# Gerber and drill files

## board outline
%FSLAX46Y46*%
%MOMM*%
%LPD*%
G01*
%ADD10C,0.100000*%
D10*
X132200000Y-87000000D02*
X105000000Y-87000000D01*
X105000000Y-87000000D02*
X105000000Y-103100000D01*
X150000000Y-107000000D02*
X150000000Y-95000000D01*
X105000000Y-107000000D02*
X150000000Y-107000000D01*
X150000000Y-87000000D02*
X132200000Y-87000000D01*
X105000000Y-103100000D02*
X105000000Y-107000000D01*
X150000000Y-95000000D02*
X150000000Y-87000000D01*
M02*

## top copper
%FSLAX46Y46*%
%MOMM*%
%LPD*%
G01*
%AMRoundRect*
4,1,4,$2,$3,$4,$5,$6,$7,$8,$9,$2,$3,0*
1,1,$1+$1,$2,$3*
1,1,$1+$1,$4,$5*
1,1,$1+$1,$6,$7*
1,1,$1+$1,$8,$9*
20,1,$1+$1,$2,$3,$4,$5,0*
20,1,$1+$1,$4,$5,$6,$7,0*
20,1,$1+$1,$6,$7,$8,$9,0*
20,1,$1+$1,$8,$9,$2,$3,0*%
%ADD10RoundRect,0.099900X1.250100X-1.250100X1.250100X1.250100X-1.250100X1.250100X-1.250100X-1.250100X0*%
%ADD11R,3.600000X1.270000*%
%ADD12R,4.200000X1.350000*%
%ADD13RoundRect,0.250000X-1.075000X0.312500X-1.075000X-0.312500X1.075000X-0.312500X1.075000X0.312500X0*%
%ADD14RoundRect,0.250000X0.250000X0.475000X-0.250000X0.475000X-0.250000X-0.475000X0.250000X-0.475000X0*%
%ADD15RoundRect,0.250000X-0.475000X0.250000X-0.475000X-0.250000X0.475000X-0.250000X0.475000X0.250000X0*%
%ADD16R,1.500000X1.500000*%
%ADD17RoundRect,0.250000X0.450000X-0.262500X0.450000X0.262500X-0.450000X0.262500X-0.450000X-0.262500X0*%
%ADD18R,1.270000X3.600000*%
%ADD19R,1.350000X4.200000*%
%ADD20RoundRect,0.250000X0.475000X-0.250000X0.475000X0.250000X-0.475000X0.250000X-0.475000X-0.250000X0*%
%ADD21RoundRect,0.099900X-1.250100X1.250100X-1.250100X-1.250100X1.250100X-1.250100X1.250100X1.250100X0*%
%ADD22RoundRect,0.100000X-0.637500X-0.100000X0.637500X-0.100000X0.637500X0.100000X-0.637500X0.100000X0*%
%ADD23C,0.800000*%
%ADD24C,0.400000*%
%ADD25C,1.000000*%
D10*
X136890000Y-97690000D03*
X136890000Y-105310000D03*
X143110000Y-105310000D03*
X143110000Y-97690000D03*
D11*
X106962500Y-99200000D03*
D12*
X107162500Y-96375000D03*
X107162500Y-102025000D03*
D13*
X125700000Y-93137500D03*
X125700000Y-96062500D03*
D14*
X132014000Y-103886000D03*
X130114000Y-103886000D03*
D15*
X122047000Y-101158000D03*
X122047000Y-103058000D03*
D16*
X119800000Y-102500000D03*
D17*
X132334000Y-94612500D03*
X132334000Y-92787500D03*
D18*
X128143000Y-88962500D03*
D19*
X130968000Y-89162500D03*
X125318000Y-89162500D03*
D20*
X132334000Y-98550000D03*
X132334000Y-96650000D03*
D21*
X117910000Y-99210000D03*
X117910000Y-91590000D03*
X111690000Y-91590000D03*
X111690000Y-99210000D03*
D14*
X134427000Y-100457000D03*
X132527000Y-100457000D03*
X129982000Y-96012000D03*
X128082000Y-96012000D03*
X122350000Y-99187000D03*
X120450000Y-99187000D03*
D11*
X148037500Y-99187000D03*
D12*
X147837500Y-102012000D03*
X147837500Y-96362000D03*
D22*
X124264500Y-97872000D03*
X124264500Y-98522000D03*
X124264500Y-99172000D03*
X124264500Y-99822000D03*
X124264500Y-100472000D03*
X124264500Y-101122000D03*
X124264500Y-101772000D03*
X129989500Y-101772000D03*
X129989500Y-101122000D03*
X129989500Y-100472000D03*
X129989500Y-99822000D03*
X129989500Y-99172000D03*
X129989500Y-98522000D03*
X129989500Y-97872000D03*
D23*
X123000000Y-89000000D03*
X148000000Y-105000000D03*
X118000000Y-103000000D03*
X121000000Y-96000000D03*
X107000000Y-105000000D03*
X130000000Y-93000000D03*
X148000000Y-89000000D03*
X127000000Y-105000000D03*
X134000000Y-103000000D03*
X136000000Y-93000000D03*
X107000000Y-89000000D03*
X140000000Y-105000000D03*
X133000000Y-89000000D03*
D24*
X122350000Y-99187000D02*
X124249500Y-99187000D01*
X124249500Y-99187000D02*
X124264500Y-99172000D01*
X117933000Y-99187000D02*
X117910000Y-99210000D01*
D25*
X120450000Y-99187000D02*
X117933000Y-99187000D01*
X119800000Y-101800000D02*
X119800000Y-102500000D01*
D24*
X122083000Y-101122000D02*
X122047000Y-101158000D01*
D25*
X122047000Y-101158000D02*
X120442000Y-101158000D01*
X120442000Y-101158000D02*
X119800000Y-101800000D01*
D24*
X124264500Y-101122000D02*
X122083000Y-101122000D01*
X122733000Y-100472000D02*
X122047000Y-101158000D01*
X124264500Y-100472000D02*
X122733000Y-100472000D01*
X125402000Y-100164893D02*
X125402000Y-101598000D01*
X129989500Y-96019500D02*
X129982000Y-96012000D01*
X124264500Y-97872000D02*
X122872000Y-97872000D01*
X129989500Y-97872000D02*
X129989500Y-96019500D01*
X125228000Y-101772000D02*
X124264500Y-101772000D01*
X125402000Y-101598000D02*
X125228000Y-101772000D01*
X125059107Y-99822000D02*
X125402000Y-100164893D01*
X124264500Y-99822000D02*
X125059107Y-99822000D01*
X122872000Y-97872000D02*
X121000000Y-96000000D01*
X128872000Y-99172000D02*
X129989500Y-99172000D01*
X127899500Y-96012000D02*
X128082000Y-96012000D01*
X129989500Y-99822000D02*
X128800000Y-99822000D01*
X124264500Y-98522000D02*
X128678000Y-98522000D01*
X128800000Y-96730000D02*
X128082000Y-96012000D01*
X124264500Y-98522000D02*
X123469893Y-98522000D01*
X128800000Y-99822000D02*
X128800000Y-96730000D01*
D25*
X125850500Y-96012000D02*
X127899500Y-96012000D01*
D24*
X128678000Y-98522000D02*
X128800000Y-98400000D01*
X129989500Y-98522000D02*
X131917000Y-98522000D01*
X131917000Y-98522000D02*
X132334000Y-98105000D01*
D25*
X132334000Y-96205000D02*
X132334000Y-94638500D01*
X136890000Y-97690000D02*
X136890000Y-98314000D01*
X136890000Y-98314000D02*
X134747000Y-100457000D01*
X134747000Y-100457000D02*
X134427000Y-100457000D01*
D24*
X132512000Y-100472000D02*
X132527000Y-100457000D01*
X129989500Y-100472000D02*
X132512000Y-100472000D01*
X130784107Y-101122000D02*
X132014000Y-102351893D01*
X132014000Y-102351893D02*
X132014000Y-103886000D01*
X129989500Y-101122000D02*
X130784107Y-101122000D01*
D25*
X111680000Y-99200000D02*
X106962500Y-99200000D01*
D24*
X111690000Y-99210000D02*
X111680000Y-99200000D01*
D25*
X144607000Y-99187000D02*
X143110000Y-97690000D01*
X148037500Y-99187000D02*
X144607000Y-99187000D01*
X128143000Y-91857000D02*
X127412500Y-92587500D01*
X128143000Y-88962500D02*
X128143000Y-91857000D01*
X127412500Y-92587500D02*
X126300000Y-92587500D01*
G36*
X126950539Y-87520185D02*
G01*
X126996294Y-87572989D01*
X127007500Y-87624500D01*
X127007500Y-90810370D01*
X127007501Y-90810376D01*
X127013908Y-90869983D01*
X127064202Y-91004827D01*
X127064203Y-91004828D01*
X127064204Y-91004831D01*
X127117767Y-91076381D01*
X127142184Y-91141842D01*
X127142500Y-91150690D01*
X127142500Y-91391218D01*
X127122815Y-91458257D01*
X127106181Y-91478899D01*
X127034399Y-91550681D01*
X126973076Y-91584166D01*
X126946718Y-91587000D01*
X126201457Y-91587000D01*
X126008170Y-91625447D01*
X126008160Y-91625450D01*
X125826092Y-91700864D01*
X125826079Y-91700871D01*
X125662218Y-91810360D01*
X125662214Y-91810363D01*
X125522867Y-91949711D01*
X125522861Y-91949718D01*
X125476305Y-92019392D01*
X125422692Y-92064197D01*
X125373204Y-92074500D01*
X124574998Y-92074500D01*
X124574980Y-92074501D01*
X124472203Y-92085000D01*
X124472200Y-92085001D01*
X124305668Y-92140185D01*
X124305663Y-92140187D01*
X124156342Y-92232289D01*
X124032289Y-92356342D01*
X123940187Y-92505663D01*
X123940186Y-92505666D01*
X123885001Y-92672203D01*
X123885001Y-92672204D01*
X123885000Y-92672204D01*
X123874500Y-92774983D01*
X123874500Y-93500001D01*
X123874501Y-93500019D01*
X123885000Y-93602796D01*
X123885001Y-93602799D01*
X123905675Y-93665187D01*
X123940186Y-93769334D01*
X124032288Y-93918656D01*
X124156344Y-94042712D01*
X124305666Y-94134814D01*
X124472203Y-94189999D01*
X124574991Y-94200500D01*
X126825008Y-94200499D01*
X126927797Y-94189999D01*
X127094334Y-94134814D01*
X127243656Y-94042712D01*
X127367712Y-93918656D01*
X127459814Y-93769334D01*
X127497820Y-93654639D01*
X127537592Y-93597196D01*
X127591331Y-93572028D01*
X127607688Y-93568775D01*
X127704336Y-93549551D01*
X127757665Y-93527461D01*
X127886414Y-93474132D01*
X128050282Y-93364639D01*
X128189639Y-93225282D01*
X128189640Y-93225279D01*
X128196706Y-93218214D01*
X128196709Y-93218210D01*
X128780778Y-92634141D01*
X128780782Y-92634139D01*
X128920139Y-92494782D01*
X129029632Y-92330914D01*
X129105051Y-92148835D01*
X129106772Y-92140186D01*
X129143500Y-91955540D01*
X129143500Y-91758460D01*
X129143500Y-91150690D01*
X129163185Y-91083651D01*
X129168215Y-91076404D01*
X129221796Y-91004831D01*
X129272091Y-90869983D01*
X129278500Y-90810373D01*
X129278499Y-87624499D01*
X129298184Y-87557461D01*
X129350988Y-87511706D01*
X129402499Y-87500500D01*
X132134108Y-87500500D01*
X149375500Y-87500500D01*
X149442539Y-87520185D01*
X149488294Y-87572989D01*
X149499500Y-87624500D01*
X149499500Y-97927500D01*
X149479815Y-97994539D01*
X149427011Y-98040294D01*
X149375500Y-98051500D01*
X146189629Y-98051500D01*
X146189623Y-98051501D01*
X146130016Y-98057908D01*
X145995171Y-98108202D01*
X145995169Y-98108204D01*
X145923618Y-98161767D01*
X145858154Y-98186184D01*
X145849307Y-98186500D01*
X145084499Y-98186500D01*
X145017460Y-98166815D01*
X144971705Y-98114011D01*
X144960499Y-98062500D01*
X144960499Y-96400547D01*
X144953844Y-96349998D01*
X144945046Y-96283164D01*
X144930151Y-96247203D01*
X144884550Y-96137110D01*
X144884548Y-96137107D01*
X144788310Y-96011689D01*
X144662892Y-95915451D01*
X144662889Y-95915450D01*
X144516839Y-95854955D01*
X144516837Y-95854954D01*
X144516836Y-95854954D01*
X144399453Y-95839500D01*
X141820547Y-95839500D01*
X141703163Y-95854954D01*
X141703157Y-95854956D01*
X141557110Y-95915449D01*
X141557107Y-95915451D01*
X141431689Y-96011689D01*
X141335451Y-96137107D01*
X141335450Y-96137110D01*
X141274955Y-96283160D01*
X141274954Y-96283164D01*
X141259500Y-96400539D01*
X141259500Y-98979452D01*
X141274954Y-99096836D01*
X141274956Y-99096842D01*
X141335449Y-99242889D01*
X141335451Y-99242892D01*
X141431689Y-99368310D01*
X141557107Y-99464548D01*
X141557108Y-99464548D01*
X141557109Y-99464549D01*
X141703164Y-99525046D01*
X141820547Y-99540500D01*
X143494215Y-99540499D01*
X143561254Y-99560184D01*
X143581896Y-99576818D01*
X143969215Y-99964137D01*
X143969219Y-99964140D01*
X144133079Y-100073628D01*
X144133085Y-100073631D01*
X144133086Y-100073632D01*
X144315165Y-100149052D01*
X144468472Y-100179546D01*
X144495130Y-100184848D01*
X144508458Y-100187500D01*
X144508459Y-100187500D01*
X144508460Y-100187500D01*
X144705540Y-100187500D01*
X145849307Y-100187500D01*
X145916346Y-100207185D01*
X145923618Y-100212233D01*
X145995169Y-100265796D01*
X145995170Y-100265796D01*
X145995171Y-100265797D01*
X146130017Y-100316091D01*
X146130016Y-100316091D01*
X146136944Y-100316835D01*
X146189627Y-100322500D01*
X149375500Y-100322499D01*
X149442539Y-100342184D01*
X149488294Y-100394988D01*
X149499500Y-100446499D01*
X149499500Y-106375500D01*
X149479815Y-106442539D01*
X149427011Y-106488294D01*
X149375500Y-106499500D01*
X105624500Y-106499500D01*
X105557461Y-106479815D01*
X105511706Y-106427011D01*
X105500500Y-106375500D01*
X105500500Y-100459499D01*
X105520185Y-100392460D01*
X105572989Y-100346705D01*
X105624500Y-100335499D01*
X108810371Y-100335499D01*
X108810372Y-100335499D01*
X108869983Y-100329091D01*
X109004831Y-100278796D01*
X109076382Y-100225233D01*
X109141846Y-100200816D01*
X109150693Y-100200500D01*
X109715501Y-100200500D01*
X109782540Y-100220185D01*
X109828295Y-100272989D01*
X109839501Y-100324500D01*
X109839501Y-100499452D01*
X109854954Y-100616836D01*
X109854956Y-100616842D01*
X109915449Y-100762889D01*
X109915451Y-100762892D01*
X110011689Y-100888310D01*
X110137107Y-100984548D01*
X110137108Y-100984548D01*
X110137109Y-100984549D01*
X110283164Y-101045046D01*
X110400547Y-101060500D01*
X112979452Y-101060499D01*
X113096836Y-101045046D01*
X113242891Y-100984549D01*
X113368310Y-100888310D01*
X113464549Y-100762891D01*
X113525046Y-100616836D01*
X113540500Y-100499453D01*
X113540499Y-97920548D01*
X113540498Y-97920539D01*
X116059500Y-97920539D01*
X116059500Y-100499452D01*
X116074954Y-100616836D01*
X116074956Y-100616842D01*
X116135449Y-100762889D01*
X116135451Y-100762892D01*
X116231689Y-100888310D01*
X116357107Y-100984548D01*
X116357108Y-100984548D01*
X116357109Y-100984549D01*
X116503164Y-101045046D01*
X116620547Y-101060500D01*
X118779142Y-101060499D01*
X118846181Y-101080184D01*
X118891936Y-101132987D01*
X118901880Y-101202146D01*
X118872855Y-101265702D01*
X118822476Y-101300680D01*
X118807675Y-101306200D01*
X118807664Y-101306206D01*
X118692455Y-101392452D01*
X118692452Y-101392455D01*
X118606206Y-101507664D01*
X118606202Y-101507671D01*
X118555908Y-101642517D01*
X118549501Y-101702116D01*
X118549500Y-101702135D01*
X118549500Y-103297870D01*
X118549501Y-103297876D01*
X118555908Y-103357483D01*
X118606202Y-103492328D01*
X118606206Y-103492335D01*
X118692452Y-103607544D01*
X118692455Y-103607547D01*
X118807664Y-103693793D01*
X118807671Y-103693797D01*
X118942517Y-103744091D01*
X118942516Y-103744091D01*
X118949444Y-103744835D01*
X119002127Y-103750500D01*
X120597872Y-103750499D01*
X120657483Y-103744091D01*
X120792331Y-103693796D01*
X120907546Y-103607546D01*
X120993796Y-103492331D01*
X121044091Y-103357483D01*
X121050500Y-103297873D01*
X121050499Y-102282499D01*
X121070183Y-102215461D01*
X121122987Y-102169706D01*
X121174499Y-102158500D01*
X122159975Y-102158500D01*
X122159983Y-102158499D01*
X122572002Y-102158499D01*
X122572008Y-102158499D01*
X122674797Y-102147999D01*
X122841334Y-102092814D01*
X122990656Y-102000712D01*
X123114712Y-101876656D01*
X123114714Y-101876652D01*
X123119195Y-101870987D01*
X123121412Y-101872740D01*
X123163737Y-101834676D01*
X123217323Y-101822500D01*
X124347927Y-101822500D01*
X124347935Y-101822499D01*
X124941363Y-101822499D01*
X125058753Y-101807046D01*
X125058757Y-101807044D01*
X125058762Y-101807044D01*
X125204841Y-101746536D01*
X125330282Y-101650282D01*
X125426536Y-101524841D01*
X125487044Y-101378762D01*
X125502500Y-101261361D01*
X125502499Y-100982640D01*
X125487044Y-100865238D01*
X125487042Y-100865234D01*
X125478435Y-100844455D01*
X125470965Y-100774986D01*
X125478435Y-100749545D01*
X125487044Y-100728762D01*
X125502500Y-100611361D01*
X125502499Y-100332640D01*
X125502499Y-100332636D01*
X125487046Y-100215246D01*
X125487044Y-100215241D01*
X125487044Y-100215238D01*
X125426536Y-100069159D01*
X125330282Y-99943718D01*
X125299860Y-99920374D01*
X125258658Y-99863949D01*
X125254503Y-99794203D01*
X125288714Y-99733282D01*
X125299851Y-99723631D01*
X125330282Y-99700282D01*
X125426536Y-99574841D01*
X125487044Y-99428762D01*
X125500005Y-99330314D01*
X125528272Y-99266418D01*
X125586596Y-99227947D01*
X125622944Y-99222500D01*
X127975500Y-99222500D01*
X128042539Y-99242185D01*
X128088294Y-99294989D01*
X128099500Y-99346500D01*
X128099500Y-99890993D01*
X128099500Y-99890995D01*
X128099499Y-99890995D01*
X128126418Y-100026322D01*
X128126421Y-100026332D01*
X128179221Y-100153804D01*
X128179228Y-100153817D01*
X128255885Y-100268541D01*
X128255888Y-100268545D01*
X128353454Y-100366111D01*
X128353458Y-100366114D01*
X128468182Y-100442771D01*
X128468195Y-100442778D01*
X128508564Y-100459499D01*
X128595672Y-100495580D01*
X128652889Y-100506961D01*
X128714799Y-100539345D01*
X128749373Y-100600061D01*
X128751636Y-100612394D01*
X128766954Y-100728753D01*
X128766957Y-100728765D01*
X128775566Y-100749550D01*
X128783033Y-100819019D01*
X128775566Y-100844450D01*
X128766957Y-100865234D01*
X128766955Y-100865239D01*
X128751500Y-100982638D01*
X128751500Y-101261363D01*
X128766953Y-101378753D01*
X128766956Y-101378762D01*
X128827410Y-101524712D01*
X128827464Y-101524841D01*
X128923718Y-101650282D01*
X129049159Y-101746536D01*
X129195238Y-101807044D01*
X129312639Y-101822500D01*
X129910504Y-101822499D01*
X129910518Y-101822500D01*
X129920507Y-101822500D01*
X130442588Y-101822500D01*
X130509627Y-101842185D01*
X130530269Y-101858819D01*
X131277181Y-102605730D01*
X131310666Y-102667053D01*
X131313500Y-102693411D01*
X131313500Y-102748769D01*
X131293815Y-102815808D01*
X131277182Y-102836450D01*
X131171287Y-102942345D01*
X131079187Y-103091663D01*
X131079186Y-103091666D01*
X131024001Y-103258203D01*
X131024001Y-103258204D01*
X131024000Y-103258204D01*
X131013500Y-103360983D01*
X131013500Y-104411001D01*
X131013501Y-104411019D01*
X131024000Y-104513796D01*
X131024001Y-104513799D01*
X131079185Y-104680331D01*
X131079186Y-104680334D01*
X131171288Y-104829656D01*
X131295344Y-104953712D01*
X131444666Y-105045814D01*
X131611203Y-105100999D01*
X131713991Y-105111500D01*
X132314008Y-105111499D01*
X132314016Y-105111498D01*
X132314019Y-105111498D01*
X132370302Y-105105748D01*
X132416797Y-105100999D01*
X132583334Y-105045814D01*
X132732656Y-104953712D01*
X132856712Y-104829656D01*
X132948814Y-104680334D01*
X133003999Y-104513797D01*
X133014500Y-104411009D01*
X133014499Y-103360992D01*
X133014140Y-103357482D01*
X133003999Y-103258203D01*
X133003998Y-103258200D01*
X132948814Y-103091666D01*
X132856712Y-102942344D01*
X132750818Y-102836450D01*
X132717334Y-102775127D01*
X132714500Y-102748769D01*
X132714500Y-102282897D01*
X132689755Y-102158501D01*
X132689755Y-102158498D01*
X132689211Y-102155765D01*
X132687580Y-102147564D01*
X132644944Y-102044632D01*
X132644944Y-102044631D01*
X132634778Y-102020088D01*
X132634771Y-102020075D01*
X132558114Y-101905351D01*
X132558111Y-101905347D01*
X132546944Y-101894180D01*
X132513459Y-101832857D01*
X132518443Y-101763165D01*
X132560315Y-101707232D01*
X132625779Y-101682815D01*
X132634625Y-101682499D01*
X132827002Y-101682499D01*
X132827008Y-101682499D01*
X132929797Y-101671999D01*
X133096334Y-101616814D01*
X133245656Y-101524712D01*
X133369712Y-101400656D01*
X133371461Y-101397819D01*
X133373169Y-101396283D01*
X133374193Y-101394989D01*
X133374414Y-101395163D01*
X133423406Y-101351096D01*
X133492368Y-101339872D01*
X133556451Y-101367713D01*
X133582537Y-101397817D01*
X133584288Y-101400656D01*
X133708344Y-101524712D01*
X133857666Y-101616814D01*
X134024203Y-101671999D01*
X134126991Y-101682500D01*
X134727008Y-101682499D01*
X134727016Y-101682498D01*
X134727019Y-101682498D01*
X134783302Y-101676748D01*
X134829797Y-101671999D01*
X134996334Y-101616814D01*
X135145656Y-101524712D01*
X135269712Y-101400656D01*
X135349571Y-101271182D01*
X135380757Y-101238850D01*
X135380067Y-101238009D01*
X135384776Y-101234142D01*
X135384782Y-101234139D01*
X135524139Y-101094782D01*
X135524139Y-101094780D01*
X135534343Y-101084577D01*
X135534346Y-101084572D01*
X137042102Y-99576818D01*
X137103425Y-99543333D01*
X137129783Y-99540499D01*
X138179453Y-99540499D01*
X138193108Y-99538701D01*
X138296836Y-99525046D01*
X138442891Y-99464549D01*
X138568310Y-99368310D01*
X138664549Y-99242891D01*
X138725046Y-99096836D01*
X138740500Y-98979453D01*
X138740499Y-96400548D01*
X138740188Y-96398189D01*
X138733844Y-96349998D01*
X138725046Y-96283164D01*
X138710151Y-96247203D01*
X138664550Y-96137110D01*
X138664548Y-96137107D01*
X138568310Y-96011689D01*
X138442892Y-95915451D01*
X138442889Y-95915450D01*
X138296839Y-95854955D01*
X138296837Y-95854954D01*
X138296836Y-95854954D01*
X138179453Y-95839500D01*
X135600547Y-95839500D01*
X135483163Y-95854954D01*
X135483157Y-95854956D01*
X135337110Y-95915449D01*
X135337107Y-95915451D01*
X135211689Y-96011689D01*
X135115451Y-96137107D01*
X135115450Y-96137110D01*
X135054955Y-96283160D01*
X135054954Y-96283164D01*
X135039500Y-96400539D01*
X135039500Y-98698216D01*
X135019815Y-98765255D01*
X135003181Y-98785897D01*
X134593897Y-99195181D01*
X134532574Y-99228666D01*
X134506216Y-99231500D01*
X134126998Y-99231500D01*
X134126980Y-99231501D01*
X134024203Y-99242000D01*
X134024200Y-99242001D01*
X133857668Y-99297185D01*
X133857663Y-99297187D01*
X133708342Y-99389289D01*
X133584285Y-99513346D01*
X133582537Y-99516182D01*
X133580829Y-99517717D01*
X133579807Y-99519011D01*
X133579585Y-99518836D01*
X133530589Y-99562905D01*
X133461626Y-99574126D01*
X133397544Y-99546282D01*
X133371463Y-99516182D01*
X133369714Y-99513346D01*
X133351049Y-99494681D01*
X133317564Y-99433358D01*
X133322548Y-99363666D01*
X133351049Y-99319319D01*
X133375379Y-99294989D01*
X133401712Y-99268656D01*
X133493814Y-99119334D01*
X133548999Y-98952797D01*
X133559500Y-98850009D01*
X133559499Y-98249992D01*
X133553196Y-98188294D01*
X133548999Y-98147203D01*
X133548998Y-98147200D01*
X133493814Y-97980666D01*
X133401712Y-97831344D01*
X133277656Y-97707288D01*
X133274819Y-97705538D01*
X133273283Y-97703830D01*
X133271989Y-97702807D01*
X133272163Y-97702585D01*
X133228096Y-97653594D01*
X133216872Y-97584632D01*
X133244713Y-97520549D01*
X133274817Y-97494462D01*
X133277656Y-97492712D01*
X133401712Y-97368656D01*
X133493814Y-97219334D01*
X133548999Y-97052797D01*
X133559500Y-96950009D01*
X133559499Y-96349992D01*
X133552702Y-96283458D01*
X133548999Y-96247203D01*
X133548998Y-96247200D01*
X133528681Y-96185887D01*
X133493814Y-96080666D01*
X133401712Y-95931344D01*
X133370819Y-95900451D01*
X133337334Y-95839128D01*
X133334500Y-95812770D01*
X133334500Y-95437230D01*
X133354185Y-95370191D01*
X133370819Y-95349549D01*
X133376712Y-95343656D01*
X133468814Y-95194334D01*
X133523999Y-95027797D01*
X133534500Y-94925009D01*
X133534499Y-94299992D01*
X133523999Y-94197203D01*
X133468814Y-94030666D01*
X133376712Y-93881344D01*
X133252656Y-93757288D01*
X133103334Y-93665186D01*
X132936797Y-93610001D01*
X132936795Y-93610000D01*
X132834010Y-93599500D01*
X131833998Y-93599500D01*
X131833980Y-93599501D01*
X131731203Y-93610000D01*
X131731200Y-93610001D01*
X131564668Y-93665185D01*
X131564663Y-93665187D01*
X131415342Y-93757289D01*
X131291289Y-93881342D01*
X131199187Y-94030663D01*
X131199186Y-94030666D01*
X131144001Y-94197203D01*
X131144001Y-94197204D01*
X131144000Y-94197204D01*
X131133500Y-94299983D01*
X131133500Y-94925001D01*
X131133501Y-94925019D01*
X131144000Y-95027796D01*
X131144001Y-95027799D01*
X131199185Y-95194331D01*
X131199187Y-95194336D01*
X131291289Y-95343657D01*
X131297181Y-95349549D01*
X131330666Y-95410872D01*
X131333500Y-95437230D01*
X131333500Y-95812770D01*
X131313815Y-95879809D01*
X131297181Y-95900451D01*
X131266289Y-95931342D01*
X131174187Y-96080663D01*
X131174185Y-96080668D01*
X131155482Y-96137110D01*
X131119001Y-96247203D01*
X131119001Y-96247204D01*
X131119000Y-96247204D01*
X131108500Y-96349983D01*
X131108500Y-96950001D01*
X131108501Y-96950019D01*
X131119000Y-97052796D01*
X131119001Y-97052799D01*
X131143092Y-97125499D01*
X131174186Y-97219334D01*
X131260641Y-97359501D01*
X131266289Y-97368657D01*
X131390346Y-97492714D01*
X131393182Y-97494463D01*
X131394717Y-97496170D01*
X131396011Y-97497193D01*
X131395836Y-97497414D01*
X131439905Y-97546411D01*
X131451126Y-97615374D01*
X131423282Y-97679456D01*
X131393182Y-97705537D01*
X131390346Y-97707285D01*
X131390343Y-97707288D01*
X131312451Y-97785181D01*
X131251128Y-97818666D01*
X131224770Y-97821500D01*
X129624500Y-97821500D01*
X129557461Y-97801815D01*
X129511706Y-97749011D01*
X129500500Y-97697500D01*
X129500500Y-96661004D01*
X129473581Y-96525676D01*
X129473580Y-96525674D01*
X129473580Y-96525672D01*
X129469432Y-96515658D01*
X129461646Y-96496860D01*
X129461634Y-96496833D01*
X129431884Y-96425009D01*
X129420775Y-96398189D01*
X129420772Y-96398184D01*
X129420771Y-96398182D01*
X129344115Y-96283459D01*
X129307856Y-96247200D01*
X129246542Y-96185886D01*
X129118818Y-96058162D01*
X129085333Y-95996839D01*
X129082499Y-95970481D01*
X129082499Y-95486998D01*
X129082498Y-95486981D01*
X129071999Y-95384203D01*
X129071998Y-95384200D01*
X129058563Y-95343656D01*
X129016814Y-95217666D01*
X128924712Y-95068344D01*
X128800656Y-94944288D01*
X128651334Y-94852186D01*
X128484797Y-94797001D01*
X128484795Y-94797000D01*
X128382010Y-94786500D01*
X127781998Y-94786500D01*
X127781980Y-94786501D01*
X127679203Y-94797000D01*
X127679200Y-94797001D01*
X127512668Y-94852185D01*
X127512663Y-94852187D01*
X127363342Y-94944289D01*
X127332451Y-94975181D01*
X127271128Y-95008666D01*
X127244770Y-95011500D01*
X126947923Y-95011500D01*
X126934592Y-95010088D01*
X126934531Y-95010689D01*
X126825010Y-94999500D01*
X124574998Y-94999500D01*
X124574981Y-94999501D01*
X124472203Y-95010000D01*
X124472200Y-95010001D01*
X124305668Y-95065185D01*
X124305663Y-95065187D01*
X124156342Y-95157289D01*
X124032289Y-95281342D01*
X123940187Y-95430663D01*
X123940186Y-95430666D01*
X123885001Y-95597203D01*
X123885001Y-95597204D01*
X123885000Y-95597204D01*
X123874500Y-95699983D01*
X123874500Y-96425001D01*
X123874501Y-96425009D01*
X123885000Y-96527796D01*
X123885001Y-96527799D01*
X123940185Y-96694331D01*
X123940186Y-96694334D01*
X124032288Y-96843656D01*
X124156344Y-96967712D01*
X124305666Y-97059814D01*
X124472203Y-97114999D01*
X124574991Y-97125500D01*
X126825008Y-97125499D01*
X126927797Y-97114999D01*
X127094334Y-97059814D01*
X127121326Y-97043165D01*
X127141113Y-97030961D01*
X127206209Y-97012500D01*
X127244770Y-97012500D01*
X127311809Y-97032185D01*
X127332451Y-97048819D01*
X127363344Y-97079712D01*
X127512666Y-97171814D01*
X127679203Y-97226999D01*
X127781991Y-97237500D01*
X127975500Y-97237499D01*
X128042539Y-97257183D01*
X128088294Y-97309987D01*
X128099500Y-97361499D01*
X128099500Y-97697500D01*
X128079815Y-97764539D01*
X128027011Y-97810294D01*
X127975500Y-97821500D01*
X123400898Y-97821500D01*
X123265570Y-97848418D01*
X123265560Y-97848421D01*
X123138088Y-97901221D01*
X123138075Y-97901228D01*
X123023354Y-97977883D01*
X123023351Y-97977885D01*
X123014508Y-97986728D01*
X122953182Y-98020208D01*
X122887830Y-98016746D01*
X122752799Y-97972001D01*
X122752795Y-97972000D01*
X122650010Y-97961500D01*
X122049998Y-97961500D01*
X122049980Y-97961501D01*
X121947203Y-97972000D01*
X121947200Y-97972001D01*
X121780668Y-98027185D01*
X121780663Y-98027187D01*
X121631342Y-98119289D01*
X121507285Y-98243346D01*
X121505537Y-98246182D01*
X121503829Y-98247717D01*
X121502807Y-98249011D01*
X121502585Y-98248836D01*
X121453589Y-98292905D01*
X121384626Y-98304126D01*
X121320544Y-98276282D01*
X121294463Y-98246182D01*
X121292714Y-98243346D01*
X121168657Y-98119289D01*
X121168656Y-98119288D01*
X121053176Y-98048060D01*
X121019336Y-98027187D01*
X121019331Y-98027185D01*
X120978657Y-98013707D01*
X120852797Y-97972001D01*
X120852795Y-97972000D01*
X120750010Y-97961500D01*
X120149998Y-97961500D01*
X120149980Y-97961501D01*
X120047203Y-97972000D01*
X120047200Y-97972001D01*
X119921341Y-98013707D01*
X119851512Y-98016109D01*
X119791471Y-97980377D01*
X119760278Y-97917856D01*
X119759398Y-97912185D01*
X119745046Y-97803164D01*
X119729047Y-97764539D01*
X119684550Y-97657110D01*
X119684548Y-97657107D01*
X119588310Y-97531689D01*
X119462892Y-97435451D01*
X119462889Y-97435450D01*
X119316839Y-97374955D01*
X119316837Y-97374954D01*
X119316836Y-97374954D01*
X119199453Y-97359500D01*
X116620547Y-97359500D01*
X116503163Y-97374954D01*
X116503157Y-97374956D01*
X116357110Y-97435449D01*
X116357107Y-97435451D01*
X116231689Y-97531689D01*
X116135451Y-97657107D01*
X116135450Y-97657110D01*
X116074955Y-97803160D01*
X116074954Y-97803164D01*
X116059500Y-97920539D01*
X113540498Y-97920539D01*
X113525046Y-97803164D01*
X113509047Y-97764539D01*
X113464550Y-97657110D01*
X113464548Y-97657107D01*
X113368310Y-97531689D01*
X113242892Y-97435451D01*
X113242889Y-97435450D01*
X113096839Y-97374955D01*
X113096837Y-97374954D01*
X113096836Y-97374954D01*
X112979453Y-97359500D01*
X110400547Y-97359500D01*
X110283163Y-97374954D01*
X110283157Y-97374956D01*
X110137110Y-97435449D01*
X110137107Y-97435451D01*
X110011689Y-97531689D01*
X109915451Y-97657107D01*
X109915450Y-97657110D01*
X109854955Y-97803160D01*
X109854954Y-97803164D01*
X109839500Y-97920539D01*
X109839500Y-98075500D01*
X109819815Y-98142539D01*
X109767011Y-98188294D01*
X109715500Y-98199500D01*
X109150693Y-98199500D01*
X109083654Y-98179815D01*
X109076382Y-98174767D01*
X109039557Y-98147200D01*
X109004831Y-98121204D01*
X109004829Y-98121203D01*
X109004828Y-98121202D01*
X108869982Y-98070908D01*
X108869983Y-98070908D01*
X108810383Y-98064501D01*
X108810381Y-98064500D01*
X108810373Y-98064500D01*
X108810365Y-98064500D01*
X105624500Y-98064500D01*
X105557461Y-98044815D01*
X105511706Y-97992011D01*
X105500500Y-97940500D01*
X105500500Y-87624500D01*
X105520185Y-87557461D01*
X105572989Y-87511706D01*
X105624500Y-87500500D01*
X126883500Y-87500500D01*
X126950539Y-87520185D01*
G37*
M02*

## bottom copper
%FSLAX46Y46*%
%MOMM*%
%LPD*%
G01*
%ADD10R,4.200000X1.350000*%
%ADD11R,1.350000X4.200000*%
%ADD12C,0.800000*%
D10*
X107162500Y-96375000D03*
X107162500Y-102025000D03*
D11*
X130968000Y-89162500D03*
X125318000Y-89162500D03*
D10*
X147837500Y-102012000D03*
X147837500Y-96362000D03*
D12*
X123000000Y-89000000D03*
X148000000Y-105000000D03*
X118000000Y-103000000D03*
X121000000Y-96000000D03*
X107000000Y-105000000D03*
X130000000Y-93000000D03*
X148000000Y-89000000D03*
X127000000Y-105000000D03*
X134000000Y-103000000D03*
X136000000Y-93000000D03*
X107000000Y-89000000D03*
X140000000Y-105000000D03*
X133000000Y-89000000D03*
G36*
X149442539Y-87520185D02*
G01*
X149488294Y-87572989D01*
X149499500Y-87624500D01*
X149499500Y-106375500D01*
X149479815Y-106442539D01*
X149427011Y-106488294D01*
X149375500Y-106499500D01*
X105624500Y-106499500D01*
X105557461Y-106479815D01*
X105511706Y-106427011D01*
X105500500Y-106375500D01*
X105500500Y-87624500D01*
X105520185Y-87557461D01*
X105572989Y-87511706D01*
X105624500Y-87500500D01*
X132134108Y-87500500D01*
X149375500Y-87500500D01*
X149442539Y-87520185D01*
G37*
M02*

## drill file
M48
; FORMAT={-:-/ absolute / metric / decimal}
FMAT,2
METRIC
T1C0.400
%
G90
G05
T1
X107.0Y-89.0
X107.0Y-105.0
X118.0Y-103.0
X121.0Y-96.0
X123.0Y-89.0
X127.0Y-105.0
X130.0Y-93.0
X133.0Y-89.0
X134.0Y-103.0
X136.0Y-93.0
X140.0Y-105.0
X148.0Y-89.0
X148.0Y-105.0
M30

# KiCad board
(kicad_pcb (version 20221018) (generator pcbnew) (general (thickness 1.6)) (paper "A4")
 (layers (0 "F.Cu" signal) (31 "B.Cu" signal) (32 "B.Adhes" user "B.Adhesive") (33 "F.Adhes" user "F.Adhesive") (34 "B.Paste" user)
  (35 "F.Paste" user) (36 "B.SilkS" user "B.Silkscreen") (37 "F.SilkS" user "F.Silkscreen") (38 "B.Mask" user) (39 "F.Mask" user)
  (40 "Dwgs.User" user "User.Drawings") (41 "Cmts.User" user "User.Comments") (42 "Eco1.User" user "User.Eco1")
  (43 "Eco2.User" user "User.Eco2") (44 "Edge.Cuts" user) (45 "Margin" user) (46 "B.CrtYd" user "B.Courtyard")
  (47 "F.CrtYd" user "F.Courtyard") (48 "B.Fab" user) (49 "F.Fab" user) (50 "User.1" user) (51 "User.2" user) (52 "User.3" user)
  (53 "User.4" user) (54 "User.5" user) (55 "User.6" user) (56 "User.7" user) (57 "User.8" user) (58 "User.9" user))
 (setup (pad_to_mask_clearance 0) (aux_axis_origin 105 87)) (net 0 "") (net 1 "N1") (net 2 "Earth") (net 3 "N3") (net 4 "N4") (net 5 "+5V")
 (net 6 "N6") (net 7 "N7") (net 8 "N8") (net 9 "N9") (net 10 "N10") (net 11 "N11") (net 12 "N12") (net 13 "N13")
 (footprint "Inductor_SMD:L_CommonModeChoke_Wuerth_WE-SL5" (layer "F.Cu") (at 140 101.5)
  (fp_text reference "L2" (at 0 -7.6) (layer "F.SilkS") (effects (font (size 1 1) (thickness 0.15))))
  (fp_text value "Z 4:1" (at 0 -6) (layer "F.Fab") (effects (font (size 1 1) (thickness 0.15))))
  (pad "1" smd roundrect (at -3.11 -3.81 90) (size 2.7 2.7) (layers "F.Cu" "F.Paste" "F.Mask") (roundrect_rratio 0.037) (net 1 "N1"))
  (pad "2" smd roundrect (at -3.11 3.81 90) (size 2.7 2.7) (layers "F.Cu" "F.Paste" "F.Mask") (roundrect_rratio 0.037) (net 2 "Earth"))
  (pad "3" smd roundrect (at 3.11 3.81 90) (size 2.7 2.7) (layers "F.Cu" "F.Paste" "F.Mask") (roundrect_rratio 0.037) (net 2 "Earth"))
  (pad "4" smd roundrect (at 3.11 -3.81 90) (size 2.7 2.7) (layers "F.Cu" "F.Paste" "F.Mask") (roundrect_rratio 0.037) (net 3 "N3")))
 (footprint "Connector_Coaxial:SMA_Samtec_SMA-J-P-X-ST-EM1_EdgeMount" (layer "F.Cu") (at 107.1625 99.2 -90)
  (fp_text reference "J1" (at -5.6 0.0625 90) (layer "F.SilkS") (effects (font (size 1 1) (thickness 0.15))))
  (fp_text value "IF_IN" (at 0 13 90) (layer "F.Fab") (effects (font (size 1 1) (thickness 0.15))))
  (pad "1" smd rect (at 0 0.2 270) (size 1.27 3.6) (layers "F.Cu" "F.Paste" "F.Mask") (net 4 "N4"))
  (pad "2" smd rect (at -2.825 0 270) (size 1.35 4.2) (layers "F.Cu" "F.Paste" "F.Mask") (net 2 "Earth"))
  (pad "2" smd rect (at -2.825 0 270) (size 1.35 4.2) (layers "B.Cu" "B.Paste" "B.Mask") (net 2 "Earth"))
  (pad "2" smd rect (at 2.825 0 270) (size 1.35 4.2) (layers "F.Cu" "F.Paste" "F.Mask") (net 2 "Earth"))
  (pad "2" smd rect (at 2.825 0 270) (size 1.35 4.2) (layers "B.Cu" "B.Paste" "B.Mask") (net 2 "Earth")))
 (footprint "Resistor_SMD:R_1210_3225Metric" (layer "F.Cu") (at 125.7 94.6 -90)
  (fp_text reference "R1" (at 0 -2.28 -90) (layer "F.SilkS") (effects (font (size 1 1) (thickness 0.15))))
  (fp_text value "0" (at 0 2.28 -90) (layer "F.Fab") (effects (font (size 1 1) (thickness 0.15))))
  (pad "1" smd roundrect (at -1.4625 0 270) (size 1.125 2.65) (layers "F.Cu" "F.Paste" "F.Mask") (roundrect_rratio 0.2222222222)
   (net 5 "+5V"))
  (pad "2" smd roundrect (at 1.4625 0 270) (size 1.125 2.65) (layers "F.Cu" "F.Paste" "F.Mask") (roundrect_rratio 0.2222222222) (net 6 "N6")))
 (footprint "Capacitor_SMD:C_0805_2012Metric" (layer "F.Cu") (at 131.064 103.886 180)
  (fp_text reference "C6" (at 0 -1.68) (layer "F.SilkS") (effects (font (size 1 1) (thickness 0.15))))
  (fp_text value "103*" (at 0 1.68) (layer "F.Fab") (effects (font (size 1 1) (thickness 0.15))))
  (pad "1" smd roundrect (at -0.95 0 180) (size 1 1.45) (layers "F.Cu" "F.Paste" "F.Mask") (roundrect_rratio 0.25) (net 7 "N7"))
  (pad "2" smd roundrect (at 0.95 0 180) (size 1 1.45) (layers "F.Cu" "F.Paste" "F.Mask") (roundrect_rratio 0.25) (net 2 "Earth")))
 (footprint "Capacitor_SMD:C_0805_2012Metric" (layer "F.Cu") (at 122.047 102.108 -90)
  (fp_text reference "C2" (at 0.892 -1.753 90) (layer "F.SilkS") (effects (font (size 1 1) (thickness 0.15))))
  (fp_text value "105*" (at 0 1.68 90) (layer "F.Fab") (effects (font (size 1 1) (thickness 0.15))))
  (pad "1" smd roundrect (at -0.95 0 270) (size 1 1.45) (layers "F.Cu" "F.Paste" "F.Mask") (roundrect_rratio 0.25) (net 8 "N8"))
  (pad "2" smd roundrect (at 0.95 0 270) (size 1 1.45) (layers "F.Cu" "F.Paste" "F.Mask") (roundrect_rratio 0.25) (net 2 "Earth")))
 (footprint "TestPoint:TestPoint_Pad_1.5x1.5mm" (layer "F.Cu") (at 119.8 102.5)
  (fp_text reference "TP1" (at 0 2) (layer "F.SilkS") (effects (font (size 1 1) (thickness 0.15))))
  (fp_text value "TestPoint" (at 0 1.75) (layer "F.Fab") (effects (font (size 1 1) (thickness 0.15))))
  (pad "1" smd rect (at 0 0) (size 1.5 1.5) (layers "F.Cu" "F.Mask") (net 8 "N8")))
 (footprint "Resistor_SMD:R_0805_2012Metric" (layer "F.Cu") (at 132.334 93.7 90)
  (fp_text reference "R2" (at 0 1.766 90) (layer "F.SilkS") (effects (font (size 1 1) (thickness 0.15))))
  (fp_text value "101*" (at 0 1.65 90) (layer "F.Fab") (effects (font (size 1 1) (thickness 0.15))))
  (pad "1" smd roundrect (at -0.9125 0 90) (size 1.025 1.4) (layers "F.Cu" "F.Paste" "F.Mask") (roundrect_rratio 0.243902439) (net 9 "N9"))
  (pad "2" smd roundrect (at 0.9125 0 90) (size 1.025 1.4) (layers "F.Cu" "F.Paste" "F.Mask") (roundrect_rratio 0.243902439) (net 2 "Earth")))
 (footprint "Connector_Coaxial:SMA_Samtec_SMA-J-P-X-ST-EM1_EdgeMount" (layer "F.Cu") (at 128.143 89.1625 180)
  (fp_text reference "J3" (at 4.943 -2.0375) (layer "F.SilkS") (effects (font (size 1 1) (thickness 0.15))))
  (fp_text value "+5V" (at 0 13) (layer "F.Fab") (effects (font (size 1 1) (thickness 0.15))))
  (pad "1" smd rect (at 0 0.2 180) (size 1.27 3.6) (layers "F.Cu" "F.Paste" "F.Mask") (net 5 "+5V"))
  (pad "2" smd rect (at -2.825 0 180) (size 1.35 4.2) (layers "F.Cu" "F.Paste" "F.Mask") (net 2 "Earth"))
  (pad "2" smd rect (at -2.825 0 180) (size 1.35 4.2) (layers "B.Cu" "B.Paste" "B.Mask") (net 2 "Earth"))
  (pad "2" smd rect (at 2.825 0 180) (size 1.35 4.2) (layers "F.Cu" "F.Paste" "F.Mask") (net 2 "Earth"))
  (pad "2" smd rect (at 2.825 0 180) (size 1.35 4.2) (layers "B.Cu" "B.Paste" "B.Mask") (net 2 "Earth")))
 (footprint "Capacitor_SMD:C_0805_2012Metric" (layer "F.Cu") (at 132.334 97.6 90)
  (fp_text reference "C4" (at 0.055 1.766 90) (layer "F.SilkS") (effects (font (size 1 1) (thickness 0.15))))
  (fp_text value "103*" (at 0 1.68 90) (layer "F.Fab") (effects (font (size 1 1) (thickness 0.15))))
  (pad "1" smd roundrect (at -0.95 0 90) (size 1 1.45) (layers "F.Cu" "F.Paste" "F.Mask") (roundrect_rratio 0.25) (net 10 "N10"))
  (pad "2" smd roundrect (at 0.95 0 90) (size 1 1.45) (layers "F.Cu" "F.Paste" "F.Mask") (roundrect_rratio 0.25) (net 9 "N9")))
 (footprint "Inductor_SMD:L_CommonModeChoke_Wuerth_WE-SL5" (layer "F.Cu") (at 114.8 95.4 180)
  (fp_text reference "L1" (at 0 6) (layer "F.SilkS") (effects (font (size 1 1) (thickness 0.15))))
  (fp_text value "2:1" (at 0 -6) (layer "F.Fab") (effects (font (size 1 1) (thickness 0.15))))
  (pad "1" smd roundrect (at -3.11 -3.81 270) (size 2.7 2.7) (layers "F.Cu" "F.Paste" "F.Mask") (roundrect_rratio 0.037) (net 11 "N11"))
  (pad "2" smd roundrect (at -3.11 3.81 270) (size 2.7 2.7) (layers "F.Cu" "F.Paste" "F.Mask") (roundrect_rratio 0.037) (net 2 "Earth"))
  (pad "3" smd roundrect (at 3.11 3.81 270) (size 2.7 2.7) (layers "F.Cu" "F.Paste" "F.Mask") (roundrect_rratio 0.037) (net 2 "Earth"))
  (pad "4" smd roundrect (at 3.11 -3.81 270) (size 2.7 2.7) (layers "F.Cu" "F.Paste" "F.Mask") (roundrect_rratio 0.037) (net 4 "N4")))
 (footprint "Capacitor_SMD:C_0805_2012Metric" (layer "F.Cu") (at 133.477 100.457 180)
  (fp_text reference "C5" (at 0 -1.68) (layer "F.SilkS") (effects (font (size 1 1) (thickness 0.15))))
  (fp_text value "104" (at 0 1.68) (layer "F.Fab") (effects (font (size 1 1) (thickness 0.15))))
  (pad "1" smd roundrect (at -0.95 0 180) (size 1 1.45) (layers "F.Cu" "F.Paste" "F.Mask") (roundrect_rratio 0.25) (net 1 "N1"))
  (pad "2" smd roundrect (at 0.95 0 180) (size 1 1.45) (layers "F.Cu" "F.Paste" "F.Mask") (roundrect_rratio 0.25) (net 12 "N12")))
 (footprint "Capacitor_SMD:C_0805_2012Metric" (layer "F.Cu") (at 129.032 96.012 180)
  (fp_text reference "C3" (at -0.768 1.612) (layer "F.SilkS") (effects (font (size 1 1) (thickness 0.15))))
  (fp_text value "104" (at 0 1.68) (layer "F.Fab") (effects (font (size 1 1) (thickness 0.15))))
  (pad "1" smd roundrect (at -0.95 0 180) (size 1 1.45) (layers "F.Cu" "F.Paste" "F.Mask") (roundrect_rratio 0.25) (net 2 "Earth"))
  (pad "2" smd roundrect (at 0.95 0 180) (size 1 1.45) (layers "F.Cu" "F.Paste" "F.Mask") (roundrect_rratio 0.25) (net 6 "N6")))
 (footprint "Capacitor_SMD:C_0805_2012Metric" (layer "F.Cu") (at 121.4 99.187 180)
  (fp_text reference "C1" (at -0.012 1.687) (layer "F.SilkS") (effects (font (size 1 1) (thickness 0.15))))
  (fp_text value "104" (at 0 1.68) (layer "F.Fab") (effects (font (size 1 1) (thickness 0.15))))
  (pad "1" smd roundrect (at -0.95 0 180) (size 1 1.45) (layers "F.Cu" "F.Paste" "F.Mask") (roundrect_rratio 0.25) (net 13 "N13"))
  (pad "2" smd roundrect (at 0.95 0 180) (size 1 1.45) (layers "F.Cu" "F.Paste" "F.Mask") (roundrect_rratio 0.25) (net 11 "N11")))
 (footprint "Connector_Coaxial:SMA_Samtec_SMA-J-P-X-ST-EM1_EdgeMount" (layer "F.Cu") (at 147.8375 99.187 90)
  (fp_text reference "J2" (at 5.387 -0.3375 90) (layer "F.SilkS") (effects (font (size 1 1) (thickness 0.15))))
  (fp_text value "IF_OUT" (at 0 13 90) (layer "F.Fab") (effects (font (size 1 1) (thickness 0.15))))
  (pad "1" smd rect (at 0 0.2 90) (size 1.27 3.6) (layers "F.Cu" "F.Paste" "F.Mask") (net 3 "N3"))
  (pad "2" smd rect (at -2.825 0 90) (size 1.35 4.2) (layers "F.Cu" "F.Paste" "F.Mask") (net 2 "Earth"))
  (pad "2" smd rect (at -2.825 0 90) (size 1.35 4.2) (layers "B.Cu" "B.Paste" "B.Mask") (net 2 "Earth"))
  (pad "2" smd rect (at 2.825 0 90) (size 1.35 4.2) (layers "F.Cu" "F.Paste" "F.Mask") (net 2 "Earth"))
  (pad "2" smd rect (at 2.825 0 90) (size 1.35 4.2) (layers "B.Cu" "B.Paste" "B.Mask") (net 2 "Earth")))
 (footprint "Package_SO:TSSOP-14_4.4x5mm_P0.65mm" (layer "F.Cu") (at 127.127 99.822)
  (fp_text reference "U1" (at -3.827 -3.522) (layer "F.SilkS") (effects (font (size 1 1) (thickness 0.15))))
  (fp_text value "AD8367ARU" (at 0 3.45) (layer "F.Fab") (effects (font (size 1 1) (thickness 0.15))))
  (pad "1" smd roundrect (at -2.8625 -1.95) (size 1.475 0.4) (layers "F.Cu" "F.Paste" "F.Mask") (roundrect_rratio 0.25) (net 2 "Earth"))
  (pad "2" smd roundrect (at -2.8625 -1.3) (size 1.475 0.4) (layers "F.Cu" "F.Paste" "F.Mask") (roundrect_rratio 0.25) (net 6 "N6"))
  (pad "3" smd roundrect (at -2.8625 -0.65) (size 1.475 0.4) (layers "F.Cu" "F.Paste" "F.Mask") (roundrect_rratio 0.25) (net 13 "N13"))
  (pad "4" smd roundrect (at -2.8625 0) (size 1.475 0.4) (layers "F.Cu" "F.Paste" "F.Mask") (roundrect_rratio 0.25) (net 2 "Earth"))
  (pad "5" smd roundrect (at -2.8625 0.65) (size 1.475 0.4) (layers "F.Cu" "F.Paste" "F.Mask") (roundrect_rratio 0.25) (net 8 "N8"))
  (pad "6" smd roundrect (at -2.8625 1.3) (size 1.475 0.4) (layers "F.Cu" "F.Paste" "F.Mask") (roundrect_rratio 0.25) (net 8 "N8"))
  (pad "7" smd roundrect (at -2.8625 1.95) (size 1.475 0.4) (layers "F.Cu" "F.Paste" "F.Mask") (roundrect_rratio 0.25) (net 2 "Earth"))
  (pad "8" smd roundrect (at 2.8625 1.95) (size 1.475 0.4) (layers "F.Cu" "F.Paste" "F.Mask") (roundrect_rratio 0.25) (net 2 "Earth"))
  (pad "9" smd roundrect (at 2.8625 1.3) (size 1.475 0.4) (layers "F.Cu" "F.Paste" "F.Mask") (roundrect_rratio 0.25) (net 7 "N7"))
  (pad "10" smd roundrect (at 2.8625 0.65) (size 1.475 0.4) (layers "F.Cu" "F.Paste" "F.Mask") (roundrect_rratio 0.25) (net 12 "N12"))
  (pad "11" smd roundrect (at 2.8625 0) (size 1.475 0.4) (layers "F.Cu" "F.Paste" "F.Mask") (roundrect_rratio 0.25) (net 6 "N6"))
  (pad "12" smd roundrect (at 2.8625 -0.65) (size 1.475 0.4) (layers "F.Cu" "F.Paste" "F.Mask") (roundrect_rratio 0.25) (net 6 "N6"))
  (pad "13" smd roundrect (at 2.8625 -1.3) (size 1.475 0.4) (layers "F.Cu" "F.Paste" "F.Mask") (roundrect_rratio 0.25) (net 10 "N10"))
  (pad "14" smd roundrect (at 2.8625 -1.95) (size 1.475 0.4) (layers "F.Cu" "F.Paste" "F.Mask") (roundrect_rratio 0.25) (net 2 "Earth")))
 (gr_line (start 132.2 87) (end 105 87) (stroke (width 0.1) (type default)) (layer "Edge.Cuts"))
 (gr_line (start 105 87) (end 105 103.1) (stroke (width 0.1) (type default)) (layer "Edge.Cuts"))
 (gr_line (start 150 107) (end 150 95) (stroke (width 0.1) (type default)) (layer "Edge.Cuts"))
 (gr_line (start 105 107) (end 150 107) (stroke (width 0.1) (type default)) (layer "Edge.Cuts"))
 (gr_line (start 150 87) (end 132.2 87) (stroke (width 0.1) (type default)) (layer "Edge.Cuts"))
 (gr_line (start 105 103.1) (end 105 107) (stroke (width 0.1) (type default)) (layer "Edge.Cuts"))
 (gr_line (start 150 95) (end 150 87) (stroke (width 0.1) (type default)) (layer "Edge.Cuts"))
 (segment (start 122.35 99.187) (end 124.2495 99.187) (width 0.4) (layer "F.Cu") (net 13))
 (segment (start 124.2495 99.187) (end 124.2645 99.172) (width 0.4) (layer "F.Cu") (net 13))
 (segment (start 117.933 99.187) (end 117.91 99.21) (width 0.4) (layer "F.Cu") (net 11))
 (segment (start 120.45 99.187) (end 117.933 99.187) (width 1) (layer "F.Cu") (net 11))
 (segment (start 119.8 101.8) (end 119.8 102.5) (width 1) (layer "F.Cu") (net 8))
 (segment (start 122.083 101.122) (end 122.047 101.158) (width 0.4) (layer "F.Cu") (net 8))
 (segment (start 122.047 101.158) (end 120.442 101.158) (width 1) (layer "F.Cu") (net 8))
 (segment (start 120.442 101.158) (end 119.8 101.8) (width 1) (layer "F.Cu") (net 8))
 (segment (start 124.2645 101.122) (end 122.083 101.122) (width 0.4) (layer "F.Cu") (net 8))
 (segment (start 122.733 100.472) (end 122.047 101.158) (width 0.4) (layer "F.Cu") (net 8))
 (segment (start 124.2645 100.472) (end 122.733 100.472) (width 0.4) (layer "F.Cu") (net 8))
 (segment (start 125.402 100.164893) (end 125.402 101.598) (width 0.4) (layer "F.Cu") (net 2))
 (segment (start 129.9895 96.0195) (end 129.982 96.012) (width 0.4) (layer "F.Cu") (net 2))
 (segment (start 124.2645 97.872) (end 122.872 97.872) (width 0.4) (layer "F.Cu") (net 2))
 (segment (start 129.9895 97.872) (end 129.9895 96.0195) (width 0.4) (layer "F.Cu") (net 2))
 (segment (start 125.228 101.772) (end 124.2645 101.772) (width 0.4) (layer "F.Cu") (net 2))
 (segment (start 125.402 101.598) (end 125.228 101.772) (width 0.4) (layer "F.Cu") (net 2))
 (segment (start 125.059107 99.822) (end 125.402 100.164893) (width 0.4) (layer "F.Cu") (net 2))
 (segment (start 124.2645 99.822) (end 125.059107 99.822) (width 0.4) (layer "F.Cu") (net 2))
 (segment (start 122.872 97.872) (end 121 96) (width 0.4) (layer "F.Cu") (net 2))
 (via (at 123 89) (size 0.8) (drill 0.4) (layers "F.Cu" "B.Cu") (free) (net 2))
 (via (at 148 105) (size 0.8) (drill 0.4) (layers "F.Cu" "B.Cu") (free) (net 2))
 (via (at 118 103) (size 0.8) (drill 0.4) (layers "F.Cu" "B.Cu") (free) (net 2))
 (via (at 121 96) (size 0.8) (drill 0.4) (layers "F.Cu" "B.Cu") (free) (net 2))
 (via (at 107 105) (size 0.8) (drill 0.4) (layers "F.Cu" "B.Cu") (free) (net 2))
 (via (at 130 93) (size 0.8) (drill 0.4) (layers "F.Cu" "B.Cu") (free) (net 2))
 (via (at 148 89) (size 0.8) (drill 0.4) (layers "F.Cu" "B.Cu") (free) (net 2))
 (via (at 127 105) (size 0.8) (drill 0.4) (layers "F.Cu" "B.Cu") (free) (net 2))
 (via (at 134 103) (size 0.8) (drill 0.4) (layers "F.Cu" "B.Cu") (free) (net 2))
 (via (at 136 93) (size 0.8) (drill 0.4) (layers "F.Cu" "B.Cu") (free) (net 2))
 (via (at 107 89) (size 0.8) (drill 0.4) (layers "F.Cu" "B.Cu") (free) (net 2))
 (via (at 140 105) (size 0.8) (drill 0.4) (layers "F.Cu" "B.Cu") (free) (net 2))
 (via (at 133 89) (size 0.8) (drill 0.4) (layers "F.Cu" "B.Cu") (free) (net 2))
 (segment (start 128.872 99.172) (end 129.9895 99.172) (width 0.4) (layer "F.Cu") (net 6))
 (segment (start 127.8995 96.012) (end 128.082 96.012) (width 0.4) (layer "F.Cu") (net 6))
 (segment (start 129.9895 99.822) (end 128.8 99.822) (width 0.4) (layer "F.Cu") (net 6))
 (segment (start 124.2645 98.522) (end 128.678 98.522) (width 0.4) (layer "F.Cu") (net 6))
 (segment (start 128.8 96.73) (end 128.082 96.012) (width 0.4) (layer "F.Cu") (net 6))
 (segment (start 124.2645 98.522) (end 123.469893 98.522) (width 0.4) (layer "F.Cu") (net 6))
 (segment (start 128.8 99.822) (end 128.8 96.73) (width 0.4) (layer "F.Cu") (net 6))
 (segment (start 125.8505 96.012) (end 127.8995 96.012) (width 1) (layer "F.Cu") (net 6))
 (segment (start 128.678 98.522) (end 128.8 98.4) (width 0.4) (layer "F.Cu") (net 6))
 (segment (start 129.9895 98.522) (end 131.917 98.522) (width 0.4) (layer "F.Cu") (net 10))
 (segment (start 131.917 98.522) (end 132.334 98.105) (width 0.4) (layer "F.Cu") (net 10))
 (segment (start 132.334 96.205) (end 132.334 94.6385) (width 1) (layer "F.Cu") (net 9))
 (segment (start 136.89 97.69) (end 136.89 98.314) (width 1) (layer "F.Cu") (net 1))
 (segment (start 136.89 98.314) (end 134.747 100.457) (width 1) (layer "F.Cu") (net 1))
 (segment (start 134.747 100.457) (end 134.427 100.457) (width 1) (layer "F.Cu") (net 1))
 (segment (start 132.512 100.472) (end 132.527 100.457) (width 0.4) (layer "F.Cu") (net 12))
 (segment (start 129.9895 100.472) (end 132.512 100.472) (width 0.4) (layer "F.Cu") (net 12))
 (segment (start 130.784107 101.122) (end 132.014 102.351893) (width 0.4) (layer "F.Cu") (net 7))
 (segment (start 132.014 102.351893) (end 132.014 103.886) (width 0.4) (layer "F.Cu") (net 7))
 (segment (start 129.9895 101.122) (end 130.784107 101.122) (width 0.4) (layer "F.Cu") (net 7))
 (segment (start 111.68 99.2) (end 106.9625 99.2) (width 1) (layer "F.Cu") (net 4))
 (segment (start 111.69 99.21) (end 111.68 99.2) (width 0.4) (layer "F.Cu") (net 4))
 (segment (start 144.607 99.187) (end 143.11 97.69) (width 1) (layer "F.Cu") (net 3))
 (segment (start 148.0375 99.187) (end 144.607 99.187) (width 1) (layer "F.Cu") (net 3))
 (segment (start 128.143 91.857) (end 127.4125 92.5875) (width 1) (layer "F.Cu") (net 5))
 (segment (start 128.143 88.9625) (end 128.143 91.857) (width 1) (layer "F.Cu") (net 5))
 (segment (start 127.4125 92.5875) (end 126.3 92.5875) (width 1) (layer "F.Cu") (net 5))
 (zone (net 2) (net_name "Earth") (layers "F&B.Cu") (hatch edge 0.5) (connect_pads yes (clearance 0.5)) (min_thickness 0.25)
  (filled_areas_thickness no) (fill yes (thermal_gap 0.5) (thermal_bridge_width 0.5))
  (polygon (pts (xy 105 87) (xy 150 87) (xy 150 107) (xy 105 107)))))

